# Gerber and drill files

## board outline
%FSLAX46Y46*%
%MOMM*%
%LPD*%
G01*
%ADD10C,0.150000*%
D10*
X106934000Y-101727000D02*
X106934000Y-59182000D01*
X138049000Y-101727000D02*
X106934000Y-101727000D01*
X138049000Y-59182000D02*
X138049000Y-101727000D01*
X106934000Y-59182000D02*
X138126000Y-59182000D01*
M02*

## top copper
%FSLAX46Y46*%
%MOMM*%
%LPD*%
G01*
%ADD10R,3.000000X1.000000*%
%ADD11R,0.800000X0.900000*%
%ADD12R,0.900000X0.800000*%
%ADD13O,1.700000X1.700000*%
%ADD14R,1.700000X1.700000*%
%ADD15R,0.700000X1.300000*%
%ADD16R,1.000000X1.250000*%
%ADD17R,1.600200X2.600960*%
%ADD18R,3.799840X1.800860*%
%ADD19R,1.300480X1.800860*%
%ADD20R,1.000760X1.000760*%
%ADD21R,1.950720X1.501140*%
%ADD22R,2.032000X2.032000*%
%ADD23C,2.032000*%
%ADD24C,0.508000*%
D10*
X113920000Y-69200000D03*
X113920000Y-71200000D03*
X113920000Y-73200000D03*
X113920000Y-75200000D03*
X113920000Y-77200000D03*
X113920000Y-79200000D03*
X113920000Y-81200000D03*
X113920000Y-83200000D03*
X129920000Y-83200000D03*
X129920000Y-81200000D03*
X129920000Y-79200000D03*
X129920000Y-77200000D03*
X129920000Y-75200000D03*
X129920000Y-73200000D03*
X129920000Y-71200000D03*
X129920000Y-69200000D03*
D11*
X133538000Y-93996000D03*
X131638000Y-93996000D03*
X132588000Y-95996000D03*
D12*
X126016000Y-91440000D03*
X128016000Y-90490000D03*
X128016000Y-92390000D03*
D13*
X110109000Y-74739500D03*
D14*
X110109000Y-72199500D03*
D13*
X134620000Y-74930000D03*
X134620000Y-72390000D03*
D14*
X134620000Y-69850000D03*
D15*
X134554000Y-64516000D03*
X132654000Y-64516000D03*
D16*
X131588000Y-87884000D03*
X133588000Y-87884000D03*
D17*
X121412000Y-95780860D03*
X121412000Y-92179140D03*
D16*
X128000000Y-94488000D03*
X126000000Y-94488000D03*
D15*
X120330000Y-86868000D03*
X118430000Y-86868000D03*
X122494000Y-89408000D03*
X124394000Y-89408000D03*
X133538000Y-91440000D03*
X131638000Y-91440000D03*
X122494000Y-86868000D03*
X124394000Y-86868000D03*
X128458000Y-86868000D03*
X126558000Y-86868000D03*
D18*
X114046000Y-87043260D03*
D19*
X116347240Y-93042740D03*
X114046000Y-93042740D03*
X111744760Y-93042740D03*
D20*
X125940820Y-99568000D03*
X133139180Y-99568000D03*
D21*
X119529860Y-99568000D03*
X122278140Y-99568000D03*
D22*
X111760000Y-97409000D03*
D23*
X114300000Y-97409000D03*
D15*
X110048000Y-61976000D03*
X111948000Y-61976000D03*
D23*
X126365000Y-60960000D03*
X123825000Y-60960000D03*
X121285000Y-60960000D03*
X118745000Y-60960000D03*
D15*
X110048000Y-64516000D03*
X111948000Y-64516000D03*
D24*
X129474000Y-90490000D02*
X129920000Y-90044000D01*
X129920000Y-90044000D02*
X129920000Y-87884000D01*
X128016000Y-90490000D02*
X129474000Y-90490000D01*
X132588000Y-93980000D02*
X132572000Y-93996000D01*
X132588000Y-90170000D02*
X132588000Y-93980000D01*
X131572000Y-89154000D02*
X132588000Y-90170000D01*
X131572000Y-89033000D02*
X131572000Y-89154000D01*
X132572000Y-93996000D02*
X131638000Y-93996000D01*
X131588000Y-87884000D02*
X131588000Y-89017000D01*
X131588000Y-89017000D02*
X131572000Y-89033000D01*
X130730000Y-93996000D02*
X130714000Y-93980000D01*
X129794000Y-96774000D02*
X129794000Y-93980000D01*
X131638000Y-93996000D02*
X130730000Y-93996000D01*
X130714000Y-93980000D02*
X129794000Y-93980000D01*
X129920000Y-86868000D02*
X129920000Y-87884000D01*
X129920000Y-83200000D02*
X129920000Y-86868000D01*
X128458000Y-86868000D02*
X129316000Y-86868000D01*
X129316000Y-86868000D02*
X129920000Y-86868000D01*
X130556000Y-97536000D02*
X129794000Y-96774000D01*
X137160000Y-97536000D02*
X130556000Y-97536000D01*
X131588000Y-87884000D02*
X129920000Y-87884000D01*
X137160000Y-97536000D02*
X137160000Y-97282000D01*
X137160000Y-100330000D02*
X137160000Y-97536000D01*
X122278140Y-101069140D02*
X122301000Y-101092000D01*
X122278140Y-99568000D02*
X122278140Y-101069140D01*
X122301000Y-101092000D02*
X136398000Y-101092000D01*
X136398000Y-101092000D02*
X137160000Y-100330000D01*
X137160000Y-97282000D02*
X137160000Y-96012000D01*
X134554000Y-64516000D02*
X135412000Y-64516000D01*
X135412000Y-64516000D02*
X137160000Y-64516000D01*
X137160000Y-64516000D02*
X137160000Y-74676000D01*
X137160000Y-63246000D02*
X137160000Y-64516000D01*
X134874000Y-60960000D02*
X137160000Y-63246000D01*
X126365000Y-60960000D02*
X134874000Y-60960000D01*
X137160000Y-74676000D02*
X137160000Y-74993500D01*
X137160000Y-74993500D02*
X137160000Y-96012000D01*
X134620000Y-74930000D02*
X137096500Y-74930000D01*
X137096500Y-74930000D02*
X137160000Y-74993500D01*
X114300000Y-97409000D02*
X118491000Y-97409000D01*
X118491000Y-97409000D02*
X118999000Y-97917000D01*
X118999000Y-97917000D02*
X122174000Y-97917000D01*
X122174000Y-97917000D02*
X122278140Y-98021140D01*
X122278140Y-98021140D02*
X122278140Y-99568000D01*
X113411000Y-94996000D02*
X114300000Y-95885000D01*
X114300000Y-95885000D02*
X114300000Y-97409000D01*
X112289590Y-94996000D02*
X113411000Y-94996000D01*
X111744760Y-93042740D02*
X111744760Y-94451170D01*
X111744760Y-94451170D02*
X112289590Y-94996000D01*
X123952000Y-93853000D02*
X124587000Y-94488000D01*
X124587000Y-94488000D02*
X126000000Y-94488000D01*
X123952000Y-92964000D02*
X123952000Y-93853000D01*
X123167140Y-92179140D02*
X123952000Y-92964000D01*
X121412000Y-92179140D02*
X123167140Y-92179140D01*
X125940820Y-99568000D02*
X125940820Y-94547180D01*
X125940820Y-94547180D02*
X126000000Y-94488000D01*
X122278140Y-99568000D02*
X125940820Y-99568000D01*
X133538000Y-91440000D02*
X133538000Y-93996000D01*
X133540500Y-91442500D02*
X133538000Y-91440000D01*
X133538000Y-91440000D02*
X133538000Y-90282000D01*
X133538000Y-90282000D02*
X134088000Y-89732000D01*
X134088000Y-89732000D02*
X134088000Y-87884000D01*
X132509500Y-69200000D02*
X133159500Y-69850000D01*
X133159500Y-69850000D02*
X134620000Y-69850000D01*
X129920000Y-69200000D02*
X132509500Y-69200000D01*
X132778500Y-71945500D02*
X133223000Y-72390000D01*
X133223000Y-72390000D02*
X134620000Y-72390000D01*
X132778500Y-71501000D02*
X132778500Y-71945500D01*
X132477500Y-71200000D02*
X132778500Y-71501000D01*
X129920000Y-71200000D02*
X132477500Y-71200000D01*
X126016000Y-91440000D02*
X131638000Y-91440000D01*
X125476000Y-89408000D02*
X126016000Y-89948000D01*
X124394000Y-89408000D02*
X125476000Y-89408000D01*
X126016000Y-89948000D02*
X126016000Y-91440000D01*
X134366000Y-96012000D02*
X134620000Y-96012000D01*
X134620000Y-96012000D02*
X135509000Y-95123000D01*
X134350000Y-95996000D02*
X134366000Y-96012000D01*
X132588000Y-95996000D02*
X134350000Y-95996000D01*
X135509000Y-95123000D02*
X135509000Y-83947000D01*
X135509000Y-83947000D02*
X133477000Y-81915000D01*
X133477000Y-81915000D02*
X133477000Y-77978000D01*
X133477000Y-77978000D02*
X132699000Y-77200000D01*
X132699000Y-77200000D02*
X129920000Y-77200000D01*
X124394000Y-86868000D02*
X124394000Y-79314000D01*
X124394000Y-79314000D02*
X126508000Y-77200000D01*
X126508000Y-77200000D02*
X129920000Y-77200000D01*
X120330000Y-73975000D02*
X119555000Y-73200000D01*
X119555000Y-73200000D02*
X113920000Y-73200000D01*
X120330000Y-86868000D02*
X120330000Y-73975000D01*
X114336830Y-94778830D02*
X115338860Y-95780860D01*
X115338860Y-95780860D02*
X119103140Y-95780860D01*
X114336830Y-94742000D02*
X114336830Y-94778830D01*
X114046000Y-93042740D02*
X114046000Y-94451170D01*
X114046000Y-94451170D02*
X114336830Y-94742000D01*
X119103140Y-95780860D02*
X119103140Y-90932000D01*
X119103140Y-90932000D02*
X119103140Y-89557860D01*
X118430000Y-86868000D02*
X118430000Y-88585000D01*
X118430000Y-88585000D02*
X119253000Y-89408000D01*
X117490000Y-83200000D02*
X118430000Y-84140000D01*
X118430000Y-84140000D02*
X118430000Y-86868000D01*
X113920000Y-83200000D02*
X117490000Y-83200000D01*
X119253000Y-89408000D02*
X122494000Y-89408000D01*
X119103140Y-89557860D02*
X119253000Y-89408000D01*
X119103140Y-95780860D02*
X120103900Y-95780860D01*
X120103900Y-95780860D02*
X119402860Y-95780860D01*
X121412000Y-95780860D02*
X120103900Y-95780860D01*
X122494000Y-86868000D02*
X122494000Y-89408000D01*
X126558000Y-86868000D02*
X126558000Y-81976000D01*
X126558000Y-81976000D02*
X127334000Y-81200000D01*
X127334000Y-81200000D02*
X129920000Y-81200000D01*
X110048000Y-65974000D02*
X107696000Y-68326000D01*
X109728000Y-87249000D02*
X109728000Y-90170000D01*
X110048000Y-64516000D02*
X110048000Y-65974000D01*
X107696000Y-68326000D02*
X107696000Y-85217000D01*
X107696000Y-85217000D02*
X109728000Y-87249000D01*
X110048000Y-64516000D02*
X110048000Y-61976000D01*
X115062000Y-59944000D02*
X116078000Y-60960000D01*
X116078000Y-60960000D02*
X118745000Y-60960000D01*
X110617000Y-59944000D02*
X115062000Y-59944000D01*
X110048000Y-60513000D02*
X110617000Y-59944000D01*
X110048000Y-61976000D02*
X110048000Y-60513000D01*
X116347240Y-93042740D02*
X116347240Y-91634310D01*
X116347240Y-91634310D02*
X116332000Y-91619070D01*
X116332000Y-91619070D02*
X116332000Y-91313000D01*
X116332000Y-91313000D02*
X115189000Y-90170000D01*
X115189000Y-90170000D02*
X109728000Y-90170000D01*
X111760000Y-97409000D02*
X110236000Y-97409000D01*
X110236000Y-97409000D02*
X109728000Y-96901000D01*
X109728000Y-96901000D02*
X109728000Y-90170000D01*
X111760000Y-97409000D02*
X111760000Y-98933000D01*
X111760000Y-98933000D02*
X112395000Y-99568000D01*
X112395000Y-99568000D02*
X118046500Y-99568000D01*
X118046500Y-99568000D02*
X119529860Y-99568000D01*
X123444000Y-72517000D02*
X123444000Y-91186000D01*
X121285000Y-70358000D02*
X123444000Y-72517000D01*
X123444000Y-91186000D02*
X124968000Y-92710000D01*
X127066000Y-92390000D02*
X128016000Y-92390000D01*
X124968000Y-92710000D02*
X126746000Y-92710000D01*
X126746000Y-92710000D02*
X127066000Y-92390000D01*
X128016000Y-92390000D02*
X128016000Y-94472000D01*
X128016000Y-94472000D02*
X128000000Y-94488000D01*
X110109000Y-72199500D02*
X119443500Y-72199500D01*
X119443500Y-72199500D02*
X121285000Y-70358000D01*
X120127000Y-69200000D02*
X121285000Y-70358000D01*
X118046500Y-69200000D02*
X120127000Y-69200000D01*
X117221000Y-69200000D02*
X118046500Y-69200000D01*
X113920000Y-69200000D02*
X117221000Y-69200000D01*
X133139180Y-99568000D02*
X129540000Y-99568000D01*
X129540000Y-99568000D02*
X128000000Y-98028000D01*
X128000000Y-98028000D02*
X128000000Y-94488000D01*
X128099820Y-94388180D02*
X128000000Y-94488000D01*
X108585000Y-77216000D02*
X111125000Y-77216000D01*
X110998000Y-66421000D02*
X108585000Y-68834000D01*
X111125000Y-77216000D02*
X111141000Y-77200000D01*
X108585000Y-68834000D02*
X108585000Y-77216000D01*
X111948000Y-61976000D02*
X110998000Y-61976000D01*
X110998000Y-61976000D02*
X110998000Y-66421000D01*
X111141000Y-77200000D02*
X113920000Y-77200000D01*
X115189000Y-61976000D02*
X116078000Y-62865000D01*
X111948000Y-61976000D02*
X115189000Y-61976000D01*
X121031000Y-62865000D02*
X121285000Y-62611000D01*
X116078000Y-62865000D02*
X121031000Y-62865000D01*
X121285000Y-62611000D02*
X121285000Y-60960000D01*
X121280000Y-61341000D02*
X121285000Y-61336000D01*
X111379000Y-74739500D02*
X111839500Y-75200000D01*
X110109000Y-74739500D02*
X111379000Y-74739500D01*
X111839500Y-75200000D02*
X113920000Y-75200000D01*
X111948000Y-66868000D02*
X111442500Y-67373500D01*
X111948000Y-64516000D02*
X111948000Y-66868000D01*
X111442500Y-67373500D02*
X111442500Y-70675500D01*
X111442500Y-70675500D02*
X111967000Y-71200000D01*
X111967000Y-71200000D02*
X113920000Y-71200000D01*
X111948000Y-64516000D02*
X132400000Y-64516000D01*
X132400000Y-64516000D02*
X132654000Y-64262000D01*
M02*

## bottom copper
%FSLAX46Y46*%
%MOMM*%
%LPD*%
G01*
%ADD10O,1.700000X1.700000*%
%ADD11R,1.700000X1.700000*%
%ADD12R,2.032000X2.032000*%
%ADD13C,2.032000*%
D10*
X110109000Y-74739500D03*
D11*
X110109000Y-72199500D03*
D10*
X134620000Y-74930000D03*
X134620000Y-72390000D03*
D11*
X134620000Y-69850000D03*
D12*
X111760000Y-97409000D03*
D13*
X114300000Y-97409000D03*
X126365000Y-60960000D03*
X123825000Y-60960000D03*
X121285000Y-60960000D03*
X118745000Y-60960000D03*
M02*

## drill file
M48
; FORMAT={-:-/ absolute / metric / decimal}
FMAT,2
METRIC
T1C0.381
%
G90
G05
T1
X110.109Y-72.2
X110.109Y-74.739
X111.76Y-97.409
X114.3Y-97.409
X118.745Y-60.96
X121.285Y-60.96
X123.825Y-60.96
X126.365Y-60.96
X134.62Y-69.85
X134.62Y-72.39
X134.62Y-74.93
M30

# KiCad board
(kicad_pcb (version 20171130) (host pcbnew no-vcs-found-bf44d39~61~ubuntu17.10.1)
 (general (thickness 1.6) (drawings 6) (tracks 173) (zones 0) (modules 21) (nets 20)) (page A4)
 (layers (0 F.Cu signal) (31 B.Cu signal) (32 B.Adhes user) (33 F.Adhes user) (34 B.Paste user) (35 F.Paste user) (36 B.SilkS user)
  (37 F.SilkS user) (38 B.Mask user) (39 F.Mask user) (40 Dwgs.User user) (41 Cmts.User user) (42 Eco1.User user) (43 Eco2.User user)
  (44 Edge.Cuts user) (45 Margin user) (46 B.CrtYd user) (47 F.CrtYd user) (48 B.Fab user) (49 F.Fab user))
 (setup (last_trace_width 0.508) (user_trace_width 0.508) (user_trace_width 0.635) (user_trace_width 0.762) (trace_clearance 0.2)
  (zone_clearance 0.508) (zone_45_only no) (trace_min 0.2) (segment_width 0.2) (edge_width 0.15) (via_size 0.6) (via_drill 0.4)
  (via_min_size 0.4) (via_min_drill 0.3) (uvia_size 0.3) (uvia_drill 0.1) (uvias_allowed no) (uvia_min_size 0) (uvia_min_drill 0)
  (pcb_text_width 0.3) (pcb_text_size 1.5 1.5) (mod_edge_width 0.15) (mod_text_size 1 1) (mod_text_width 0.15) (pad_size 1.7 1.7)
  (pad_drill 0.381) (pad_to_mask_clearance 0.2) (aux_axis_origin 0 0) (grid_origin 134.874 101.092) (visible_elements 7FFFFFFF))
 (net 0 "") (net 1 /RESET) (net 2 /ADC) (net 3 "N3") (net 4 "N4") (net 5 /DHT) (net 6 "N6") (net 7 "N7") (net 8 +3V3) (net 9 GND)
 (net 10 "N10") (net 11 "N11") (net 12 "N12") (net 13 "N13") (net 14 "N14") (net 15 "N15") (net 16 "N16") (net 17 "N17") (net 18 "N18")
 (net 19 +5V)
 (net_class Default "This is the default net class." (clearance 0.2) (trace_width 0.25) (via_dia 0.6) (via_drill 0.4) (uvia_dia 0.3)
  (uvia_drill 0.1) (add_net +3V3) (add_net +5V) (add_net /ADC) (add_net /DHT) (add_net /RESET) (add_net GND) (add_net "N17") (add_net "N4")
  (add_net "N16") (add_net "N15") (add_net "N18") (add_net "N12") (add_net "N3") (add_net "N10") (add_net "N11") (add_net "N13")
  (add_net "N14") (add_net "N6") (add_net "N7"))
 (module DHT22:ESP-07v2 (layer F.Cu) (at 121.92 76.2)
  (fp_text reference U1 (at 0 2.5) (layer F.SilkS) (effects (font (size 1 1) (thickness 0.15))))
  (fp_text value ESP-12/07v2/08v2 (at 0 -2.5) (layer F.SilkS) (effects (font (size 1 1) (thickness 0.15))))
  (pad 1 smd rect (at -8 -7) (size 3 1) (layers F.Cu F.Paste F.Mask) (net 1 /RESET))
  (pad 2 smd rect (at -8 -5) (size 3 1) (layers F.Cu F.Paste F.Mask) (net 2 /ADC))
  (pad 3 smd rect (at -8 -3) (size 3 1) (layers F.Cu F.Paste F.Mask) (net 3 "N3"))
  (pad 4 smd rect (at -8 -1) (size 3 1) (layers F.Cu F.Paste F.Mask) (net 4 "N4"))
  (pad 5 smd rect (at -8 1) (size 3 1) (layers F.Cu F.Paste F.Mask) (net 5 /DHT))
  (pad 6 smd rect (at -8 3) (size 3 1) (layers F.Cu F.Paste F.Mask) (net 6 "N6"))
  (pad 7 smd rect (at -8 5) (size 3 1) (layers F.Cu F.Paste F.Mask) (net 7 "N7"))
  (pad 8 smd rect (at -8 7) (size 3 1) (layers F.Cu F.Paste F.Mask) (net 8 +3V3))
  (pad 9 smd rect (at 8 7) (size 3 1) (layers F.Cu F.Paste F.Mask) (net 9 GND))
  (pad 10 smd rect (at 8 5) (size 3 1) (layers F.Cu F.Paste F.Mask) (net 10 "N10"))
  (pad 11 smd rect (at 8 3) (size 3 1) (layers F.Cu F.Paste F.Mask) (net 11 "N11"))
  (pad 12 smd rect (at 8 1) (size 3 1) (layers F.Cu F.Paste F.Mask) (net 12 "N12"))
  (pad 13 smd rect (at 8 -1) (size 3 1) (layers F.Cu F.Paste F.Mask) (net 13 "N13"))
  (pad 14 smd rect (at 8 -3) (size 3 1) (layers F.Cu F.Paste F.Mask) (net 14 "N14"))
  (pad 15 smd rect (at 8 -5) (size 3 1) (layers F.Cu F.Paste F.Mask) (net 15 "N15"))
  (pad 16 smd rect (at 8 -7) (size 3 1) (layers F.Cu F.Paste F.Mask) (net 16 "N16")))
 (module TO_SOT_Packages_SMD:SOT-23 (layer F.Cu) (at 132.588 94.996 270)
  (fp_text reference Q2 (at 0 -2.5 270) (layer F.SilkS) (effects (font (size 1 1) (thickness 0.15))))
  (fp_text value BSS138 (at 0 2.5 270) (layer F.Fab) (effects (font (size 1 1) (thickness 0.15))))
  (pad 1 smd rect (at -1 -0.95 270) (size 0.9 0.8) (layers F.Cu F.Paste F.Mask) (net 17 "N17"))
  (pad 2 smd rect (at -1 0.95 270) (size 0.9 0.8) (layers F.Cu F.Paste F.Mask) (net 9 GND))
  (pad 3 smd rect (at 1 0 270) (size 0.9 0.8) (layers F.Cu F.Paste F.Mask) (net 12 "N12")))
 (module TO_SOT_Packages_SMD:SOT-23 (layer F.Cu) (at 127.016 91.44 180)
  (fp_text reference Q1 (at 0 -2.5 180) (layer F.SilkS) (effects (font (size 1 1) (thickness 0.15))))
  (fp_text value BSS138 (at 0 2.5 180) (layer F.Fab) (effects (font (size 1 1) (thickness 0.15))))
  (pad 3 smd rect (at 1 0 180) (size 0.9 0.8) (layers F.Cu F.Paste F.Mask) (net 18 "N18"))
  (pad 2 smd rect (at -1 0.95 180) (size 0.9 0.8) (layers F.Cu F.Paste F.Mask) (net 9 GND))
  (pad 1 smd rect (at -1 -0.95 180) (size 0.9 0.8) (layers F.Cu F.Paste F.Mask) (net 1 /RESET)))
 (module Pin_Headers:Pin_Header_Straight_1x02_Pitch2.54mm (layer F.Cu) (at 110.109 72.1995)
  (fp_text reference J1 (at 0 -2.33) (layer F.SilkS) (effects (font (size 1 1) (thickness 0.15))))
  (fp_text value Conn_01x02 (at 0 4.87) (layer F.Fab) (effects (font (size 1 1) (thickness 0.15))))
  (pad 2 thru_hole oval (at 0 2.54) (size 1.7 1.7) (drill 0.381) (layers *.Cu *.Mask) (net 4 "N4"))
  (pad 1 thru_hole rect (at 0 0) (size 1.7 1.7) (drill 0.381) (layers *.Cu *.Mask) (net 1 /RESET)))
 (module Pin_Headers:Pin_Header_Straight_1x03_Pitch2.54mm (layer F.Cu) (at 134.62 69.85)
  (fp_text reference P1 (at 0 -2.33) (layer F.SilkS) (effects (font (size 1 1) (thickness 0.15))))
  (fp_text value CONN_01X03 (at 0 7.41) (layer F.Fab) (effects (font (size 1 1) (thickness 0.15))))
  (pad 3 thru_hole oval (at 0 5.08) (size 1.7 1.7) (drill 0.381) (layers *.Cu *.Mask) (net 9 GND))
  (pad 2 thru_hole oval (at 0 2.54) (size 1.7 1.7) (drill 0.381) (layers *.Cu *.Mask) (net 15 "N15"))
  (pad 1 thru_hole rect (at 0 0) (size 1.7 1.7) (drill 0.381) (layers *.Cu *.Mask) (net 16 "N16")))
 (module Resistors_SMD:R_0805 (layer F.Cu) (at 133.604 64.516)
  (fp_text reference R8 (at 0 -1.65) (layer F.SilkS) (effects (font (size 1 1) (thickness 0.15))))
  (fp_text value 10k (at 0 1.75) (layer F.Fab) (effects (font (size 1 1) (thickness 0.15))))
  (pad 2 smd rect (at 0.95 0) (size 0.7 1.3) (layers F.Cu F.Paste F.Mask) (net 9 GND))
  (pad 1 smd rect (at -0.95 0) (size 0.7 1.3) (layers F.Cu F.Paste F.Mask) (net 2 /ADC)))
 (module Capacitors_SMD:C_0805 (layer F.Cu) (at 132.588 87.884 180)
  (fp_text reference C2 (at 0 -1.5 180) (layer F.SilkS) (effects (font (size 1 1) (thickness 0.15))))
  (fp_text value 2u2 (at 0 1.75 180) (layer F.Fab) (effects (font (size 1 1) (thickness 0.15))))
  (pad 2 smd rect (at 1 0 180) (size 1 1.25) (layers F.Cu F.Paste F.Mask) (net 9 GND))
  (pad 1 smd rect (at -1 0 180) (size 1 1.25) (layers F.Cu F.Paste F.Mask) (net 17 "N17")))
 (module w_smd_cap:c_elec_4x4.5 (layer F.Cu) (at 121.412 93.98 270)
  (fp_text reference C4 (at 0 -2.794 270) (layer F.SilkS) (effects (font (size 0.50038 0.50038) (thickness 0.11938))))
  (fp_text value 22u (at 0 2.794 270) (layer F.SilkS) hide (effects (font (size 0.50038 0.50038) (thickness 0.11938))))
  (pad 1 smd rect (at 1.80086 0 270) (size 2.60096 1.6002) (layers F.Cu F.Paste F.Mask) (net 8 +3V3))
  (pad 2 smd rect (at -1.80086 0 270) (size 2.60096 1.6002) (layers F.Cu F.Paste F.Mask) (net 9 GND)))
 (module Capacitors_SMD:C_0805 (layer F.Cu) (at 127 94.488 180)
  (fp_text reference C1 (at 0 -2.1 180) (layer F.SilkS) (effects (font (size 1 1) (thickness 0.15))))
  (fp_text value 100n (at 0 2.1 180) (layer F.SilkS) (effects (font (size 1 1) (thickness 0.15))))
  (pad 1 smd rect (at -1 0 180) (size 1 1.25) (layers F.Cu F.Paste F.Mask) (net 1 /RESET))
  (pad 2 smd rect (at 1 0 180) (size 1 1.25) (layers F.Cu F.Paste F.Mask) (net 9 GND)))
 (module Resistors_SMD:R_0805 (layer F.Cu) (at 119.38 86.868 180)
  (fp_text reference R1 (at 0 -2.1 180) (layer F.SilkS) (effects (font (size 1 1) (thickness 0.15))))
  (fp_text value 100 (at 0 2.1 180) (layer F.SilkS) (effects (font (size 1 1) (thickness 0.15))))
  (pad 1 smd rect (at -0.95 0 180) (size 0.7 1.3) (layers F.Cu F.Paste F.Mask) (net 3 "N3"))
  (pad 2 smd rect (at 0.95 0 180) (size 0.7 1.3) (layers F.Cu F.Paste F.Mask) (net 8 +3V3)))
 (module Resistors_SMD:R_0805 (layer F.Cu) (at 123.444 89.408)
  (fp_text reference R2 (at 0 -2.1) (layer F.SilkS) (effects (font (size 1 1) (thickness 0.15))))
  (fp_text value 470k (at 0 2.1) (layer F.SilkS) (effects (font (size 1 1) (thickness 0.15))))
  (pad 1 smd rect (at -0.95 0) (size 0.7 1.3) (layers F.Cu F.Paste F.Mask) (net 8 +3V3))
  (pad 2 smd rect (at 0.95 0) (size 0.7 1.3) (layers F.Cu F.Paste F.Mask) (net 18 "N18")))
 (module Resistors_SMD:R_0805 (layer F.Cu) (at 132.588 91.44 180)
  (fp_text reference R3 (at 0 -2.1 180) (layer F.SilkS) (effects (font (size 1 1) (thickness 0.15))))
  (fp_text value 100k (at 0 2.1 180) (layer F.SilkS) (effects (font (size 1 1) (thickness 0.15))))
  (pad 1 smd rect (at -0.95 0 180) (size 0.7 1.3) (layers F.Cu F.Paste F.Mask) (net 17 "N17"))
  (pad 2 smd rect (at 0.95 0 180) (size 0.7 1.3) (layers F.Cu F.Paste F.Mask) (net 18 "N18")))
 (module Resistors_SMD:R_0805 (layer F.Cu) (at 123.444 86.868)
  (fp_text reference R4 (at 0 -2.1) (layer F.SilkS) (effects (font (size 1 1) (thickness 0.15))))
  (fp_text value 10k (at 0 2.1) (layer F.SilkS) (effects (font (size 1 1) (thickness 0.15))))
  (pad 1 smd rect (at -0.95 0) (size 0.7 1.3) (layers F.Cu F.Paste F.Mask) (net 8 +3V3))
  (pad 2 smd rect (at 0.95 0) (size 0.7 1.3) (layers F.Cu F.Paste F.Mask) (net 12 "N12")))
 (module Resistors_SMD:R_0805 (layer F.Cu) (at 127.508 86.868 180)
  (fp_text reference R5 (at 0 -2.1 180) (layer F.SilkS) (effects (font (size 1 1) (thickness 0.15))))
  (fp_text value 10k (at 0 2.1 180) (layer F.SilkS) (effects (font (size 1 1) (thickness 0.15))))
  (pad 1 smd rect (at -0.95 0 180) (size 0.7 1.3) (layers F.Cu F.Paste F.Mask) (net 9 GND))
  (pad 2 smd rect (at 0.95 0 180) (size 0.7 1.3) (layers F.Cu F.Paste F.Mask) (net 10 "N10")))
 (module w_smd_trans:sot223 (layer F.Cu) (at 114.046 90.043)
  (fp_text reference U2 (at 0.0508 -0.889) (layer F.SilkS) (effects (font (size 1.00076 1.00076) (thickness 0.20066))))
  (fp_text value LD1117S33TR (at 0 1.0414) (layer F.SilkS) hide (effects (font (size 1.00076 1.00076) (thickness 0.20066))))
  (pad 4 smd rect (at 0 -2.99974) (size 3.79984 1.80086) (layers F.Cu F.Paste F.Mask))
  (pad 3 smd rect (at 2.30124 2.99974) (size 1.30048 1.80086) (layers F.Cu F.Paste F.Mask) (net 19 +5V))
  (pad 2 smd rect (at 0 2.99974) (size 1.30048 1.80086) (layers F.Cu F.Paste F.Mask) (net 8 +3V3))
  (pad 1 smd rect (at -2.30124 2.99974) (size 1.30048 1.80086) (layers F.Cu F.Paste F.Mask) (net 9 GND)))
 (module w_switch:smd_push (layer F.Cu) (at 129.54 99.568) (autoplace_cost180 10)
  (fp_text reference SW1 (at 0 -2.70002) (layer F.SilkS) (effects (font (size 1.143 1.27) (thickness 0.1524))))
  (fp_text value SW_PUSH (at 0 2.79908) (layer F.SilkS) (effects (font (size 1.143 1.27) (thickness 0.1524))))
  (pad 1 smd rect (at -3.59918 0) (size 1.00076 1.00076) (layers F.Cu F.Paste F.Mask) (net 9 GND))
  (pad 2 smd rect (at 3.59918 0) (size 1.00076 1.00076) (layers F.Cu F.Paste F.Mask) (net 1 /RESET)))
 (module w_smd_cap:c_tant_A (layer F.Cu) (at 120.904 99.568 180)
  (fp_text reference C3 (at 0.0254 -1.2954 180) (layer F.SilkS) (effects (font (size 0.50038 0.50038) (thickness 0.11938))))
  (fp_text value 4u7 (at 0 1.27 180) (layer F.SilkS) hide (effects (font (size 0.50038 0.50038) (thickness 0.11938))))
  (pad 1 smd rect (at 1.37414 0 180) (size 1.95072 1.50114) (layers F.Cu F.Paste F.Mask) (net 19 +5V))
  (pad 2 smd rect (at -1.37414 0 180) (size 1.95072 1.50114) (layers F.Cu F.Paste F.Mask) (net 9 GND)))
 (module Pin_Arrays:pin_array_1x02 (layer F.Cu) (at 113.03 97.409)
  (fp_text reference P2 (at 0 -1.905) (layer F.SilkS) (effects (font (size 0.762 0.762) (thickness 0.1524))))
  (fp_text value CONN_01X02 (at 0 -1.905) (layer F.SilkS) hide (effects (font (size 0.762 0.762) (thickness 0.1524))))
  (pad 1 thru_hole rect (at -1.27 0) (size 2.032 2.032) (drill 0.381) (layers *.Cu *.Mask F.SilkS) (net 19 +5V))
  (pad 2 thru_hole circle (at 1.27 0) (size 2.032 2.032) (drill 0.381) (layers *.Cu *.Mask F.SilkS) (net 9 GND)))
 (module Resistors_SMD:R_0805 (layer F.Cu) (at 110.998 61.976)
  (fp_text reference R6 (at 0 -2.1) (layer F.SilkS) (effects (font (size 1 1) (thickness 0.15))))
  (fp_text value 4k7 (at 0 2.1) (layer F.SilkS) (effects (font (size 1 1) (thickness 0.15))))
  (pad 1 smd rect (at -0.95 0) (size 0.7 1.3) (layers F.Cu F.Paste F.Mask) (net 19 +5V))
  (pad 2 smd rect (at 0.95 0) (size 0.7 1.3) (layers F.Cu F.Paste F.Mask) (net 5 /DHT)))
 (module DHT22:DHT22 (layer B.Cu) (at 122.555 77.47)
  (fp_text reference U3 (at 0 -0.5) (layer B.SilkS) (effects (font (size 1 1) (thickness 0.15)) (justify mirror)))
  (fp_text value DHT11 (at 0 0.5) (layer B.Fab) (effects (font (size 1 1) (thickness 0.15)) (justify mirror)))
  (pad 4 thru_hole circle (at 3.81 -16.51) (size 2.032 2.032) (drill 0.381) (layers *.Cu *.Mask B.SilkS) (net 9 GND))
  (pad 3 thru_hole circle (at 1.27 -16.51) (size 2.032 2.032) (drill 0.381) (layers *.Cu *.Mask B.SilkS))
  (pad 2 thru_hole circle (at -1.27 -16.51) (size 2.032 2.032) (drill 0.381) (layers *.Cu *.Mask B.SilkS) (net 5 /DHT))
  (pad 1 thru_hole circle (at -3.81 -16.51) (size 2.032 2.032) (drill 0.381) (layers *.Cu *.Mask B.SilkS) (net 19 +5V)))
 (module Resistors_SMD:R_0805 (layer F.Cu) (at 110.998 64.516)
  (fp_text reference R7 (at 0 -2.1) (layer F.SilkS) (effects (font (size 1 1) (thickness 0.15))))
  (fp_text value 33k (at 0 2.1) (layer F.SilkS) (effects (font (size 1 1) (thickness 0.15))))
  (pad 1 smd rect (at -0.95 0) (size 0.7 1.3) (layers F.Cu F.Paste F.Mask) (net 19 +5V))
  (pad 2 smd rect (at 0.95 0) (size 0.7 1.3) (layers F.Cu F.Paste F.Mask) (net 2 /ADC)))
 (gr_line (start 106.934 101.727) (end 106.934 59.182) (angle 90) (layer Edge.Cuts) (width 0.15))
 (gr_line (start 138.049 101.727) (end 106.934 101.727) (angle 90) (layer Edge.Cuts) (width 0.15))
 (gr_line (start 138.049 59.182) (end 138.049 101.727) (angle 90) (layer Edge.Cuts) (width 0.15))
 (gr_line (start 106.934 59.182) (end 138.126 59.182) (angle 90) (layer Edge.Cuts) (width 0.15))
 (segment (start 129.474 90.49) (end 129.92 90.044) (width 0.508) (layer F.Cu) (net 9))
 (segment (start 129.92 90.044) (end 129.92 87.884) (width 0.508) (layer F.Cu) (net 9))
 (segment (start 128.016 90.49) (end 129.474 90.49) (width 0.508) (layer F.Cu) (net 9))
 (segment (start 132.588 93.98) (end 132.572 93.996) (width 0.508) (layer F.Cu) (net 9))
 (segment (start 132.588 90.17) (end 132.588 93.98) (width 0.508) (layer F.Cu) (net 9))
 (segment (start 131.572 89.154) (end 132.588 90.17) (width 0.508) (layer F.Cu) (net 9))
 (segment (start 131.572 89.033) (end 131.572 89.154) (width 0.508) (layer F.Cu) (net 9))
 (segment (start 132.572 93.996) (end 131.638 93.996) (width 0.508) (layer F.Cu) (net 9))
 (segment (start 131.588 87.884) (end 131.588 89.017) (width 0.508) (layer F.Cu) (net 9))
 (segment (start 131.588 89.017) (end 131.572 89.033) (width 0.508) (layer F.Cu) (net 9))
 (segment (start 130.73 93.996) (end 130.714 93.98) (width 0.508) (layer F.Cu) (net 9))
 (segment (start 129.794 96.774) (end 129.794 93.98) (width 0.508) (layer F.Cu) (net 9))
 (segment (start 131.638 93.996) (end 130.73 93.996) (width 0.508) (layer F.Cu) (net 9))
 (segment (start 130.714 93.98) (end 129.794 93.98) (width 0.508) (layer F.Cu) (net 9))
 (segment (start 129.92 86.868) (end 129.92 87.884) (width 0.508) (layer F.Cu) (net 9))
 (segment (start 129.92 83.2) (end 129.92 86.868) (width 0.508) (layer F.Cu) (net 9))
 (segment (start 128.458 86.868) (end 129.316 86.868) (width 0.508) (layer F.Cu) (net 9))
 (segment (start 129.316 86.868) (end 129.92 86.868) (width 0.508) (layer F.Cu) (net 9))
 (segment (start 130.556 97.536) (end 129.794 96.774) (width 0.508) (layer F.Cu) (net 9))
 (segment (start 137.16 97.536) (end 130.556 97.536) (width 0.508) (layer F.Cu) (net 9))
 (segment (start 131.588 87.884) (end 129.92 87.884) (width 0.508) (layer F.Cu) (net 9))
 (segment (start 137.16 97.536) (end 137.16 97.282) (width 0.508) (layer F.Cu) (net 9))
 (segment (start 137.16 100.33) (end 137.16 97.536) (width 0.508) (layer F.Cu) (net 9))
 (segment (start 122.27814 101.06914) (end 122.301 101.092) (width 0.508) (layer F.Cu) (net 9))
 (segment (start 122.27814 99.568) (end 122.27814 101.06914) (width 0.508) (layer F.Cu) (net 9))
 (segment (start 122.301 101.092) (end 136.398 101.092) (width 0.508) (layer F.Cu) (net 9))
 (segment (start 136.398 101.092) (end 137.16 100.33) (width 0.508) (layer F.Cu) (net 9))
 (segment (start 137.16 97.282) (end 137.16 96.012) (width 0.508) (layer F.Cu) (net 9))
 (segment (start 134.554 64.516) (end 135.412 64.516) (width 0.508) (layer F.Cu) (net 9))
 (segment (start 135.412 64.516) (end 137.16 64.516) (width 0.508) (layer F.Cu) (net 9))
 (segment (start 137.16 64.516) (end 137.16 74.676) (width 0.508) (layer F.Cu) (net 9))
 (segment (start 137.16 63.246) (end 137.16 64.516) (width 0.508) (layer F.Cu) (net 9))
 (segment (start 134.874 60.96) (end 137.16 63.246) (width 0.508) (layer F.Cu) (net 9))
 (segment (start 126.365 60.96) (end 134.874 60.96) (width 0.508) (layer F.Cu) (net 9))
 (segment (start 137.16 74.676) (end 137.16 74.9935) (width 0.508) (layer F.Cu) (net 9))
 (segment (start 137.16 74.9935) (end 137.16 96.012) (width 0.508) (layer F.Cu) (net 9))
 (segment (start 134.62 74.93) (end 137.0965 74.93) (width 0.508) (layer F.Cu) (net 9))
 (segment (start 137.0965 74.93) (end 137.16 74.9935) (width 0.508) (layer F.Cu) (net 9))
 (segment (start 114.3 97.409) (end 118.491 97.409) (width 0.508) (layer F.Cu) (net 9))
 (segment (start 118.491 97.409) (end 118.999 97.917) (width 0.508) (layer F.Cu) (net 9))
 (segment (start 118.999 97.917) (end 122.174 97.917) (width 0.508) (layer F.Cu) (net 9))
 (segment (start 122.174 97.917) (end 122.27814 98.02114) (width 0.508) (layer F.Cu) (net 9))
 (segment (start 122.27814 98.02114) (end 122.27814 99.568) (width 0.508) (layer F.Cu) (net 9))
 (segment (start 113.411 94.996) (end 114.3 95.885) (width 0.508) (layer F.Cu) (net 9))
 (segment (start 114.3 95.885) (end 114.3 97.409) (width 0.508) (layer F.Cu) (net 9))
 (segment (start 112.28959 94.996) (end 113.411 94.996) (width 0.508) (layer F.Cu) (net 9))
 (segment (start 111.74476 93.04274) (end 111.74476 94.45117) (width 0.508) (layer F.Cu) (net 9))
 (segment (start 111.74476 94.45117) (end 112.28959 94.996) (width 0.508) (layer F.Cu) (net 9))
 (segment (start 123.952 93.853) (end 124.587 94.488) (width 0.508) (layer F.Cu) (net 9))
 (segment (start 124.587 94.488) (end 126 94.488) (width 0.508) (layer F.Cu) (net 9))
 (segment (start 123.952 92.964) (end 123.952 93.853) (width 0.508) (layer F.Cu) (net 9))
 (segment (start 123.16714 92.17914) (end 123.952 92.964) (width 0.508) (layer F.Cu) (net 9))
 (segment (start 121.412 92.17914) (end 123.16714 92.17914) (width 0.508) (layer F.Cu) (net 9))
 (segment (start 125.94082 99.568) (end 125.94082 94.54718) (width 0.508) (layer F.Cu) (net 9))
 (segment (start 125.94082 94.54718) (end 126 94.488) (width 0.508) (layer F.Cu) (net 9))
 (segment (start 122.27814 99.568) (end 125.94082 99.568) (width 0.508) (layer F.Cu) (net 9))
 (segment (start 133.538 91.44) (end 133.538 93.996) (width 0.508) (layer F.Cu) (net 17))
 (segment (start 133.5405 91.4425) (end 133.538 91.44) (width 0.508) (layer F.Cu) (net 17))
 (segment (start 133.538 91.44) (end 133.538 90.282) (width 0.508) (layer F.Cu) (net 17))
 (segment (start 133.538 90.282) (end 134.088 89.732) (width 0.508) (layer F.Cu) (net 17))
 (segment (start 134.088 89.732) (end 134.088 87.884) (width 0.508) (layer F.Cu) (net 17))
 (segment (start 132.5095 69.2) (end 133.1595 69.85) (width 0.508) (layer F.Cu) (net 16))
 (segment (start 133.1595 69.85) (end 134.62 69.85) (width 0.508) (layer F.Cu) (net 16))
 (segment (start 129.92 69.2) (end 132.5095 69.2) (width 0.508) (layer F.Cu) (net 16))
 (segment (start 132.7785 71.9455) (end 133.223 72.39) (width 0.508) (layer F.Cu) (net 15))
 (segment (start 133.223 72.39) (end 134.62 72.39) (width 0.508) (layer F.Cu) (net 15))
 (segment (start 132.7785 71.501) (end 132.7785 71.9455) (width 0.508) (layer F.Cu) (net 15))
 (segment (start 132.4775 71.2) (end 132.7785 71.501) (width 0.508) (layer F.Cu) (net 15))
 (segment (start 129.92 71.2) (end 132.4775 71.2) (width 0.508) (layer F.Cu) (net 15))
 (segment (start 126.016 91.44) (end 131.638 91.44) (width 0.508) (layer F.Cu) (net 18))
 (segment (start 125.476 89.408) (end 126.016 89.948) (width 0.508) (layer F.Cu) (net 18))
 (segment (start 124.394 89.408) (end 125.476 89.408) (width 0.508) (layer F.Cu) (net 18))
 (segment (start 126.016 89.948) (end 126.016 91.44) (width 0.508) (layer F.Cu) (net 18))
 (segment (start 134.366 96.012) (end 134.62 96.012) (width 0.508) (layer F.Cu) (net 12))
 (segment (start 134.62 96.012) (end 135.509 95.123) (width 0.508) (layer F.Cu) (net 12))
 (segment (start 134.35 95.996) (end 134.366 96.012) (width 0.508) (layer F.Cu) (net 12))
 (segment (start 132.588 95.996) (end 134.35 95.996) (width 0.508) (layer F.Cu) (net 12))
 (segment (start 135.509 95.123) (end 135.509 83.947) (width 0.508) (layer F.Cu) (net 12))
 (segment (start 135.509 83.947) (end 133.477 81.915) (width 0.508) (layer F.Cu) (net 12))
 (segment (start 133.477 81.915) (end 133.477 77.978) (width 0.508) (layer F.Cu) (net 12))
 (segment (start 133.477 77.978) (end 132.699 77.2) (width 0.508) (layer F.Cu) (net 12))
 (segment (start 132.699 77.2) (end 129.92 77.2) (width 0.508) (layer F.Cu) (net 12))
 (segment (start 124.394 86.868) (end 124.394 79.314) (width 0.508) (layer F.Cu) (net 12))
 (segment (start 124.394 79.314) (end 126.508 77.2) (width 0.508) (layer F.Cu) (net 12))
 (segment (start 126.508 77.2) (end 129.92 77.2) (width 0.508) (layer F.Cu) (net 12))
 (segment (start 120.33 73.975) (end 119.555 73.2) (width 0.508) (layer F.Cu) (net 3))
 (segment (start 119.555 73.2) (end 113.92 73.2) (width 0.508) (layer F.Cu) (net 3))
 (segment (start 120.33 86.868) (end 120.33 73.975) (width 0.508) (layer F.Cu) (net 3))
 (segment (start 114.33683 94.77883) (end 115.33886 95.78086) (width 0.508) (layer F.Cu) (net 8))
 (segment (start 115.33886 95.78086) (end 119.10314 95.78086) (width 0.508) (layer F.Cu) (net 8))
 (segment (start 114.33683 94.742) (end 114.33683 94.77883) (width 0.508) (layer F.Cu) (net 8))
 (segment (start 114.046 93.04274) (end 114.046 94.45117) (width 0.508) (layer F.Cu) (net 8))
 (segment (start 114.046 94.45117) (end 114.33683 94.742) (width 0.508) (layer F.Cu) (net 8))
 (segment (start 119.10314 95.78086) (end 119.10314 90.932) (width 0.508) (layer F.Cu) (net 8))
 (segment (start 119.10314 90.932) (end 119.10314 89.55786) (width 0.508) (layer F.Cu) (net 8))
 (segment (start 118.43 86.868) (end 118.43 88.585) (width 0.508) (layer F.Cu) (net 8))
 (segment (start 118.43 88.585) (end 119.253 89.408) (width 0.508) (layer F.Cu) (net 8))
 (segment (start 117.49 83.2) (end 118.43 84.14) (width 0.508) (layer F.Cu) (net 8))
 (segment (start 118.43 84.14) (end 118.43 86.868) (width 0.508) (layer F.Cu) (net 8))
 (segment (start 113.92 83.2) (end 117.49 83.2) (width 0.508) (layer F.Cu) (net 8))
 (segment (start 119.253 89.408) (end 122.494 89.408) (width 0.508) (layer F.Cu) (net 8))
 (segment (start 119.10314 89.55786) (end 119.253 89.408) (width 0.508) (layer F.Cu) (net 8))
 (segment (start 119.10314 95.78086) (end 120.1039 95.78086) (width 0.508) (layer F.Cu) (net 8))
 (segment (start 120.1039 95.78086) (end 119.40286 95.78086) (width 0.508) (layer F.Cu) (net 8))
 (segment (start 121.412 95.78086) (end 120.1039 95.78086) (width 0.508) (layer F.Cu) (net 8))
 (segment (start 122.494 86.868) (end 122.494 89.408) (width 0.508) (layer F.Cu) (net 8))
 (segment (start 126.558 86.868) (end 126.558 81.976) (width 0.508) (layer F.Cu) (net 10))
 (segment (start 126.558 81.976) (end 127.334 81.2) (width 0.508) (layer F.Cu) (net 10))
 (segment (start 127.334 81.2) (end 129.92 81.2) (width 0.508) (layer F.Cu) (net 10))
 (segment (start 110.048 65.974) (end 107.696 68.326) (width 0.508) (layer F.Cu) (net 19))
 (segment (start 109.728 87.249) (end 109.728 90.17) (width 0.508) (layer F.Cu) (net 19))
 (segment (start 110.048 64.516) (end 110.048 65.974) (width 0.508) (layer F.Cu) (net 19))
 (segment (start 107.696 68.326) (end 107.696 85.217) (width 0.508) (layer F.Cu) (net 19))
 (segment (start 107.696 85.217) (end 109.728 87.249) (width 0.508) (layer F.Cu) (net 19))
 (segment (start 110.048 64.516) (end 110.048 61.976) (width 0.508) (layer F.Cu) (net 19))
 (segment (start 115.062 59.944) (end 116.078 60.96) (width 0.508) (layer F.Cu) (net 19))
 (segment (start 116.078 60.96) (end 118.745 60.96) (width 0.508) (layer F.Cu) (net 19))
 (segment (start 110.617 59.944) (end 115.062 59.944) (width 0.508) (layer F.Cu) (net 19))
 (segment (start 110.048 60.513) (end 110.617 59.944) (width 0.508) (layer F.Cu) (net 19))
 (segment (start 110.048 61.976) (end 110.048 60.513) (width 0.508) (layer F.Cu) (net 19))
 (segment (start 116.34724 93.04274) (end 116.34724 91.63431) (width 0.508) (layer F.Cu) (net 19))
 (segment (start 116.34724 91.63431) (end 116.332 91.61907) (width 0.508) (layer F.Cu) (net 19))
 (segment (start 116.332 91.61907) (end 116.332 91.313) (width 0.508) (layer F.Cu) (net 19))
 (segment (start 116.332 91.313) (end 115.189 90.17) (width 0.508) (layer F.Cu) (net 19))
 (segment (start 115.189 90.17) (end 109.728 90.17) (width 0.508) (layer F.Cu) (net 19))
 (segment (start 111.76 97.409) (end 110.236 97.409) (width 0.508) (layer F.Cu) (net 19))
 (segment (start 110.236 97.409) (end 109.728 96.901) (width 0.508) (layer F.Cu) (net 19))
 (segment (start 109.728 96.901) (end 109.728 90.17) (width 0.508) (layer F.Cu) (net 19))
 (segment (start 111.76 97.409) (end 111.76 98.933) (width 0.508) (layer F.Cu) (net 19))
 (segment (start 111.76 98.933) (end 112.395 99.568) (width 0.508) (layer F.Cu) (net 19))
 (segment (start 112.395 99.568) (end 118.0465 99.568) (width 0.508) (layer F.Cu) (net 19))
 (segment (start 118.0465 99.568) (end 119.52986 99.568) (width 0.508) (layer F.Cu) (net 19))
 (segment (start 123.444 72.517) (end 123.444 91.186) (width 0.508) (layer F.Cu) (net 1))
 (segment (start 121.285 70.358) (end 123.444 72.517) (width 0.508) (layer F.Cu) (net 1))
 (segment (start 123.444 91.186) (end 124.968 92.71) (width 0.508) (layer F.Cu) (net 1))
 (segment (start 127.066 92.39) (end 128.016 92.39) (width 0.508) (layer F.Cu) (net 1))
 (segment (start 124.968 92.71) (end 126.746 92.71) (width 0.508) (layer F.Cu) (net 1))
 (segment (start 126.746 92.71) (end 127.066 92.39) (width 0.508) (layer F.Cu) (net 1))
 (segment (start 128.016 92.39) (end 128.016 94.472) (width 0.508) (layer F.Cu) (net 1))
 (segment (start 128.016 94.472) (end 128 94.488) (width 0.508) (layer F.Cu) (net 1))
 (segment (start 110.109 72.1995) (end 119.4435 72.1995) (width 0.508) (layer F.Cu) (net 1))
 (segment (start 119.4435 72.1995) (end 121.285 70.358) (width 0.508) (layer F.Cu) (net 1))
 (segment (start 120.127 69.2) (end 121.285 70.358) (width 0.508) (layer F.Cu) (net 1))
 (segment (start 118.0465 69.2) (end 120.127 69.2) (width 0.508) (layer F.Cu) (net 1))
 (segment (start 117.221 69.2) (end 118.0465 69.2) (width 0.508) (layer F.Cu) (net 1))
 (segment (start 113.92 69.2) (end 117.221 69.2) (width 0.508) (layer F.Cu) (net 1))
 (segment (start 133.13918 99.568) (end 129.54 99.568) (width 0.508) (layer F.Cu) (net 1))
 (segment (start 129.54 99.568) (end 128 98.028) (width 0.508) (layer F.Cu) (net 1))
 (segment (start 128 98.028) (end 128 94.488) (width 0.508) (layer F.Cu) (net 1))
 (segment (start 128.09982 94.38818) (end 128 94.488) (width 0.508) (layer F.Cu) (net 1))
 (segment (start 108.585 77.216) (end 111.125 77.216) (width 0.508) (layer F.Cu) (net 5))
 (segment (start 110.998 66.421) (end 108.585 68.834) (width 0.508) (layer F.Cu) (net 5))
 (segment (start 111.125 77.216) (end 111.141 77.2) (width 0.508) (layer F.Cu) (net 5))
 (segment (start 108.585 68.834) (end 108.585 77.216) (width 0.508) (layer F.Cu) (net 5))
 (segment (start 111.948 61.976) (end 110.998 61.976) (width 0.508) (layer F.Cu) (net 5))
 (segment (start 110.998 61.976) (end 110.998 66.421) (width 0.508) (layer F.Cu) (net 5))
 (segment (start 111.141 77.2) (end 113.92 77.2) (width 0.508) (layer F.Cu) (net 5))
 (segment (start 115.189 61.976) (end 116.078 62.865) (width 0.508) (layer F.Cu) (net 5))
 (segment (start 111.948 61.976) (end 115.189 61.976) (width 0.508) (layer F.Cu) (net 5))
 (segment (start 121.031 62.865) (end 121.285 62.611) (width 0.508) (layer F.Cu) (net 5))
 (segment (start 116.078 62.865) (end 121.031 62.865) (width 0.508) (layer F.Cu) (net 5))
 (segment (start 121.285 62.611) (end 121.285 60.96) (width 0.508) (layer F.Cu) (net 5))
 (segment (start 121.28 61.341) (end 121.285 61.336) (width 0.508) (layer F.Cu) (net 5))
 (segment (start 111.379 74.7395) (end 111.8395 75.2) (width 0.508) (layer F.Cu) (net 4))
 (segment (start 110.109 74.7395) (end 111.379 74.7395) (width 0.508) (layer F.Cu) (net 4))
 (segment (start 111.8395 75.2) (end 113.92 75.2) (width 0.508) (layer F.Cu) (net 4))
 (segment (start 111.948 66.868) (end 111.4425 67.3735) (width 0.508) (layer F.Cu) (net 2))
 (segment (start 111.948 64.516) (end 111.948 66.868) (width 0.508) (layer F.Cu) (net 2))
 (segment (start 111.4425 67.3735) (end 111.4425 70.6755) (width 0.508) (layer F.Cu) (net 2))
 (segment (start 111.4425 70.6755) (end 111.967 71.2) (width 0.508) (layer F.Cu) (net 2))
 (segment (start 111.967 71.2) (end 113.92 71.2) (width 0.508) (layer F.Cu) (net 2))
 (segment (start 111.948 64.516) (end 132.4 64.516) (width 0.508) (layer F.Cu) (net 2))
 (segment (start 132.4 64.516) (end 132.654 64.262) (width 0.508) (layer F.Cu) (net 2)))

